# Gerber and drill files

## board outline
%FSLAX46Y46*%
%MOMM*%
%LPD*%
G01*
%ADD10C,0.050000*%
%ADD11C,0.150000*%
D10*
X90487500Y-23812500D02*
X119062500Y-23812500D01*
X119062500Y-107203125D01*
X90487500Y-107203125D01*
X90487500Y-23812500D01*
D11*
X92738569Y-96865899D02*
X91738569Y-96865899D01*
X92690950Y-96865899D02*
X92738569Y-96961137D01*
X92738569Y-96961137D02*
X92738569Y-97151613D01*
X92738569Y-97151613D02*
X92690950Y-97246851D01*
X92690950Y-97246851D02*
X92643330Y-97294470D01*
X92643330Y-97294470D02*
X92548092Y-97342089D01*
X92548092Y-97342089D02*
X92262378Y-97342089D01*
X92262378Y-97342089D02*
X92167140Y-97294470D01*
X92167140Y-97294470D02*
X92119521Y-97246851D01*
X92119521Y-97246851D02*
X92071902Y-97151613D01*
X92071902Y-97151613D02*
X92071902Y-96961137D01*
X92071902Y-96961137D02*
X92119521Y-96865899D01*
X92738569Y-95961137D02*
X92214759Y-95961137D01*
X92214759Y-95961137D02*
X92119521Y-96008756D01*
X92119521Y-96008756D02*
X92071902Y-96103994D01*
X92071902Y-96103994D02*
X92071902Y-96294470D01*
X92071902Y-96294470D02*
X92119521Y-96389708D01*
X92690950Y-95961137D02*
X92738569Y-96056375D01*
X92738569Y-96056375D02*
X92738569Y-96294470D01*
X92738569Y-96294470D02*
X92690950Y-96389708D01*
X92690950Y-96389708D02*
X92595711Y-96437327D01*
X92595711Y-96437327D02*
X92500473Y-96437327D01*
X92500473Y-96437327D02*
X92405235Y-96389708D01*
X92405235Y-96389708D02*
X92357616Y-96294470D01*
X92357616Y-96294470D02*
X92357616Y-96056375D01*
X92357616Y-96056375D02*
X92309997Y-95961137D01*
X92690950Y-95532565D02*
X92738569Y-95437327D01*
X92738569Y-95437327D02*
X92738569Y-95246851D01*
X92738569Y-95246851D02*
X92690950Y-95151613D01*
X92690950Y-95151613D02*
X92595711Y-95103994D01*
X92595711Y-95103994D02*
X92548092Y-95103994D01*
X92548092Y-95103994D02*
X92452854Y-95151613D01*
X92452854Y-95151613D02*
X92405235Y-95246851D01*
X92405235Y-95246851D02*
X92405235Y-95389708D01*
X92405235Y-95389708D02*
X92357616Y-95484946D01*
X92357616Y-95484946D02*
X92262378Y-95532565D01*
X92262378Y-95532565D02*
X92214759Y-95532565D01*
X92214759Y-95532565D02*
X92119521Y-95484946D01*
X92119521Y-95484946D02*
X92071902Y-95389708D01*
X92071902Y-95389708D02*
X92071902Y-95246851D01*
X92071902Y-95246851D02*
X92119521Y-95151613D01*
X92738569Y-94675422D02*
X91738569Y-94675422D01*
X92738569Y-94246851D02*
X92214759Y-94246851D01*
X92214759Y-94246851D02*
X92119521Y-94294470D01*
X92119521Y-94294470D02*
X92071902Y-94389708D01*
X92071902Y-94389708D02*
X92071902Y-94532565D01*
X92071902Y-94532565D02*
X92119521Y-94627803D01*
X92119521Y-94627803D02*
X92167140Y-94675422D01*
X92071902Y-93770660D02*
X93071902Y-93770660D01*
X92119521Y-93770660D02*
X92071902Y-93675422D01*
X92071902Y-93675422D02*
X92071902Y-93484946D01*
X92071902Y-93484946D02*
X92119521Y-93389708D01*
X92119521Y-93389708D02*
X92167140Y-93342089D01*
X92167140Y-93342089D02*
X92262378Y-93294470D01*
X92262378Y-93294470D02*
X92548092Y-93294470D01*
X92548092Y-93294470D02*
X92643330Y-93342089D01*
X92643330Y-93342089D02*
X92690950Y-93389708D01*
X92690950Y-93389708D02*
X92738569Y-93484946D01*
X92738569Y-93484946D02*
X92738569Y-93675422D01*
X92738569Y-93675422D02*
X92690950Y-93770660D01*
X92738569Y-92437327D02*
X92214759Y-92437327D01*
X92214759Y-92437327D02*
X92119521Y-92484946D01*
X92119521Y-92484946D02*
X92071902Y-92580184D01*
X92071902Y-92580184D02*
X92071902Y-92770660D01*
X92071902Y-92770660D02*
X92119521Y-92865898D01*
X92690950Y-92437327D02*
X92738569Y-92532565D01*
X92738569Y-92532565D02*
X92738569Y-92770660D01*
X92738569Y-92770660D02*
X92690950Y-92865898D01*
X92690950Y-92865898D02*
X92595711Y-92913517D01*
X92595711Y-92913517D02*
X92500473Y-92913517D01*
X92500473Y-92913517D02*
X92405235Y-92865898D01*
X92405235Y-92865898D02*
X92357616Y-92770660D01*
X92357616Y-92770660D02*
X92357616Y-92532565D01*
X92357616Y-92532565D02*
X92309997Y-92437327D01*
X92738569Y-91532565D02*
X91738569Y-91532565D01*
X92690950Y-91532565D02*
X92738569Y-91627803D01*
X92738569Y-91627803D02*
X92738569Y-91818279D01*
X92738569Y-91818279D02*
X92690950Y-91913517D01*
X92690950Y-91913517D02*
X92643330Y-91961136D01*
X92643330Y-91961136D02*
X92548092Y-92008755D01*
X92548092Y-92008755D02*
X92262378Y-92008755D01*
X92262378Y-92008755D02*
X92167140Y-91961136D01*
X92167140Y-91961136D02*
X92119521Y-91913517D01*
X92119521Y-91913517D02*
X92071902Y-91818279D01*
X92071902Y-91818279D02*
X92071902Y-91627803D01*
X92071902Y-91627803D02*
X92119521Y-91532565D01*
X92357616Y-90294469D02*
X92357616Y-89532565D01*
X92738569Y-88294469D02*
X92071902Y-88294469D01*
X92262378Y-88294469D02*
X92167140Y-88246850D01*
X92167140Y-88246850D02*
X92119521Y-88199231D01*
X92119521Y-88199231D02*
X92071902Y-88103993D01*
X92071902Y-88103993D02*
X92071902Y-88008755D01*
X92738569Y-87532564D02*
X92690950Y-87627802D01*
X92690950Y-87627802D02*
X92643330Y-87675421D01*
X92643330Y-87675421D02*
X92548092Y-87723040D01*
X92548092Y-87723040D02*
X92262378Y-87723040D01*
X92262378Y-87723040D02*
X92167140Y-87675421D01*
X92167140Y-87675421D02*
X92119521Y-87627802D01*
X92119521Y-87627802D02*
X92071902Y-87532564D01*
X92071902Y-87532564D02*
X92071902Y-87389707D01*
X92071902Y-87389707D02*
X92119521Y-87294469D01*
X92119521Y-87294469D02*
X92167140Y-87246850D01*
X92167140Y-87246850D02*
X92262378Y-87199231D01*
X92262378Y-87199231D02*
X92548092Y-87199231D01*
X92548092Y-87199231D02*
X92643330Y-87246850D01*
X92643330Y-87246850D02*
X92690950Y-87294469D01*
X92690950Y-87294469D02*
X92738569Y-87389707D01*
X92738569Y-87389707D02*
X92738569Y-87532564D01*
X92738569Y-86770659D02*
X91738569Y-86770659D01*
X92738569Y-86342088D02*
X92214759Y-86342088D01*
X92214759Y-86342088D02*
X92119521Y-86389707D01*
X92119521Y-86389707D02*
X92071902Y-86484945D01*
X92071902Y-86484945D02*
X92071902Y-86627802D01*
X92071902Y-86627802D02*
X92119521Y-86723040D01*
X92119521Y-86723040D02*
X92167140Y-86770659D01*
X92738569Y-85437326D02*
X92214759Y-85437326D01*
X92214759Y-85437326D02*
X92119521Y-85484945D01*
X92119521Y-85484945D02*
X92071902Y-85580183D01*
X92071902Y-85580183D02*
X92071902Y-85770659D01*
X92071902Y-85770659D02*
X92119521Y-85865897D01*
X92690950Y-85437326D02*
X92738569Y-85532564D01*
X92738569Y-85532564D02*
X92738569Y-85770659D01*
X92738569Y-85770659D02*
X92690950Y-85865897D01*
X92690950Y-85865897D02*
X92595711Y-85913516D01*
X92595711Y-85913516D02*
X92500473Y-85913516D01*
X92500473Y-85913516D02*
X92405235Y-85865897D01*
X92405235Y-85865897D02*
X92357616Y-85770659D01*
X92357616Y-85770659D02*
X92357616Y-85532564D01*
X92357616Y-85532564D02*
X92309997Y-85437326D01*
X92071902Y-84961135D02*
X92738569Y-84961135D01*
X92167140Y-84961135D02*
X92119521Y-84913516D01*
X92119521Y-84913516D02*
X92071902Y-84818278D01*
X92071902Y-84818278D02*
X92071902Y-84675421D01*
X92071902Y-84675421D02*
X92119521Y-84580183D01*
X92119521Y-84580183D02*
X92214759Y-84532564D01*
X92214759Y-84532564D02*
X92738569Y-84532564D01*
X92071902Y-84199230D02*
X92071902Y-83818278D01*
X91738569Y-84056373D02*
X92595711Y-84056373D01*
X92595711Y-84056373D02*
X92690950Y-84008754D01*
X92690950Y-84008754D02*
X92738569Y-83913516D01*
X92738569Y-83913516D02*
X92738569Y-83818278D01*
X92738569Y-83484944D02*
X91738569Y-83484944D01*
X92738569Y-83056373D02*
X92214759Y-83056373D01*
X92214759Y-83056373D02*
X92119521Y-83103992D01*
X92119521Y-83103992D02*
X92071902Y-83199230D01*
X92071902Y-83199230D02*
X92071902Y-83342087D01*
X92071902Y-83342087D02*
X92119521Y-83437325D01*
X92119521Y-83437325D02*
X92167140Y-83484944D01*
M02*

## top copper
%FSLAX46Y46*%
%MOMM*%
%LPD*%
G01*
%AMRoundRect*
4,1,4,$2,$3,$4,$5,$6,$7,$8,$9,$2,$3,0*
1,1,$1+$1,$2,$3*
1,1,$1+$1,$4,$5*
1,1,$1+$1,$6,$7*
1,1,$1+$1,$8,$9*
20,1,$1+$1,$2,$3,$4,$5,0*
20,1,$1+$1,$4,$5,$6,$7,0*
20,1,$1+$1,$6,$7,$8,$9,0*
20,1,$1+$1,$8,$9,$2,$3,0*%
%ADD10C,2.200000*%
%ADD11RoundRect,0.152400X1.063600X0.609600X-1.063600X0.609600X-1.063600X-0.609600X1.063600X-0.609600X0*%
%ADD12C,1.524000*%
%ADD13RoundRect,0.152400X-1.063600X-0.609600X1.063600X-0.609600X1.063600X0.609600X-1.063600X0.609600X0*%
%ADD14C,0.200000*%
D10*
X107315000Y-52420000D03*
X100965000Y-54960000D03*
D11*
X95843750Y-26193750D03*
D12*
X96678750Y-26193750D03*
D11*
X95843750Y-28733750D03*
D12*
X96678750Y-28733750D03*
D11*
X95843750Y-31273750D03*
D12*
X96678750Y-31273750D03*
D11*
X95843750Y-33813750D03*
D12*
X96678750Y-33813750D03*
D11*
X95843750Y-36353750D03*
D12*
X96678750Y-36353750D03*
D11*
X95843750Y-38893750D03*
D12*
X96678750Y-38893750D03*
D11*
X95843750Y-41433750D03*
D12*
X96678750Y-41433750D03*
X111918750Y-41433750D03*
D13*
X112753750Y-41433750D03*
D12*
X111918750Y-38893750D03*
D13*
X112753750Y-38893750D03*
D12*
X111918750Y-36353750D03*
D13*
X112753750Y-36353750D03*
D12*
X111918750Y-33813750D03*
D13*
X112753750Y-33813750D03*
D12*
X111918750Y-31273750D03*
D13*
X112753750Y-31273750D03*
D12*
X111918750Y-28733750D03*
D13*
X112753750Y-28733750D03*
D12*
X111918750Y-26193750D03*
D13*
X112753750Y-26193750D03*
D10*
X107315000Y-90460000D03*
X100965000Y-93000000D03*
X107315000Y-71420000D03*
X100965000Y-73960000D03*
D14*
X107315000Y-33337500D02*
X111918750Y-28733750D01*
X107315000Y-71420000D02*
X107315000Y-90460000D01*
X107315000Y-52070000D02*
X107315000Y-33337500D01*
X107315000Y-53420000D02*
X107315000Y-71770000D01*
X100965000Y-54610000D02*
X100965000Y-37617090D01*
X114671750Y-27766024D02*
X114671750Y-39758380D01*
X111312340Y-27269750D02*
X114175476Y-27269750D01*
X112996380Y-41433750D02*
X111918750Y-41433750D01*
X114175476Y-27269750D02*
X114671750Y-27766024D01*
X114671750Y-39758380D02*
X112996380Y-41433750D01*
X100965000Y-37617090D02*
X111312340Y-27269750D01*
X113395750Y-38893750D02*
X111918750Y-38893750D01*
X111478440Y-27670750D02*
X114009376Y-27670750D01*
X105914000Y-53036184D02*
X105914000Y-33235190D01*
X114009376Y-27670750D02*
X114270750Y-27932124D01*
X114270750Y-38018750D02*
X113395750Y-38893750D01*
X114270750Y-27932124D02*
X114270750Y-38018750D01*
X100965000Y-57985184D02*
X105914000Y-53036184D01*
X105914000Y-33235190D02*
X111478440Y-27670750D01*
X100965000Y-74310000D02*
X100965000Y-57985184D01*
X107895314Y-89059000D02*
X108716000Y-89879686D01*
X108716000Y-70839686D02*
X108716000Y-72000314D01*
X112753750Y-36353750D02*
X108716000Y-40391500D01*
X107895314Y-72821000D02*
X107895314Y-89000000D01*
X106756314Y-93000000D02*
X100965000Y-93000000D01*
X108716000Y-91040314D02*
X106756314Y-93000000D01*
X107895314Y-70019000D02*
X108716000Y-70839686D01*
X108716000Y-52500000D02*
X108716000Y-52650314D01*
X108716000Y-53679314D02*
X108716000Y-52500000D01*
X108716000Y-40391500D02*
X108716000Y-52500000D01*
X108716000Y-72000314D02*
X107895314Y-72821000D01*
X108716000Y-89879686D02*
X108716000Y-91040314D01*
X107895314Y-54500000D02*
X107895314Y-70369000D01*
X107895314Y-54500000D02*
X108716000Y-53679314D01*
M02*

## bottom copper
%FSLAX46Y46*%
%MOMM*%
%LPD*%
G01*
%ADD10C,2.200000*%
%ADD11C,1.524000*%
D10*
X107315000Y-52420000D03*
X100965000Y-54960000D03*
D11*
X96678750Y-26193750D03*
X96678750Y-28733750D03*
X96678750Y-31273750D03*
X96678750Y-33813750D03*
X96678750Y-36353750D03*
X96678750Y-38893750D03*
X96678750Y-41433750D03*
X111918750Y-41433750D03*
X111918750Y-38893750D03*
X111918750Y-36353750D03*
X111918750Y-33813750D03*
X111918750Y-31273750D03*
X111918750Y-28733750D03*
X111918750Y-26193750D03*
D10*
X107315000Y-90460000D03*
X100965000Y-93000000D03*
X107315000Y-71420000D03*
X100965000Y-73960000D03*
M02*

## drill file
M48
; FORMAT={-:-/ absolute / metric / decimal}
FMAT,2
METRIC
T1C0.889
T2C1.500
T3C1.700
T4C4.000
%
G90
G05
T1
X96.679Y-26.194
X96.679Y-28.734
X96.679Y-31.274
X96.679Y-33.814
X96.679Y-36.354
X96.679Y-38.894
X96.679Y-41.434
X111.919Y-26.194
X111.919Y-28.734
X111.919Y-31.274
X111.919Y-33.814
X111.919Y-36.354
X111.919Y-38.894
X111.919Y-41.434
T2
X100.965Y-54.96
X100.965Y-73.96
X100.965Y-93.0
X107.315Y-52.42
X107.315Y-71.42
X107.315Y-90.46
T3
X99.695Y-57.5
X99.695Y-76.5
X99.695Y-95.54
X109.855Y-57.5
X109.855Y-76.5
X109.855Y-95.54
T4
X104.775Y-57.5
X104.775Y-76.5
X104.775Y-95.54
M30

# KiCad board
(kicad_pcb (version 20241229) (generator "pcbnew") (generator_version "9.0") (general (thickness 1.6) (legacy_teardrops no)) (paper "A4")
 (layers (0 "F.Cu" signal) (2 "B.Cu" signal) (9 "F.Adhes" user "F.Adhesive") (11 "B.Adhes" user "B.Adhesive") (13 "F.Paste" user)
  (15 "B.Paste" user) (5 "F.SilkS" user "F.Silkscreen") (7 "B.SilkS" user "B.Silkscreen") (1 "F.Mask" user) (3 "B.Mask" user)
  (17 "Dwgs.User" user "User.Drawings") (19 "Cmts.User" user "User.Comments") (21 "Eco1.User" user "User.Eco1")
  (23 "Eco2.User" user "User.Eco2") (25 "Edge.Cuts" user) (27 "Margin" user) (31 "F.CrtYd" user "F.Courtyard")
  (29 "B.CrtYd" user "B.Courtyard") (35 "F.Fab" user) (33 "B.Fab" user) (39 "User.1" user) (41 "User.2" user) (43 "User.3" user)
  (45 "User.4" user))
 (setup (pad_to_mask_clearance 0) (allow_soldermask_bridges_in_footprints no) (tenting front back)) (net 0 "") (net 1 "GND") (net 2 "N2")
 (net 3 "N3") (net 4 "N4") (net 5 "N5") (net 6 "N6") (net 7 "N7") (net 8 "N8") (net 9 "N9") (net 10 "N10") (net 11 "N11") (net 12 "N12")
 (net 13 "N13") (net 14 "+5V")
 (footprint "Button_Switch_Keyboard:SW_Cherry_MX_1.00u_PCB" (layer "F.Cu") (at 107.315 52.42)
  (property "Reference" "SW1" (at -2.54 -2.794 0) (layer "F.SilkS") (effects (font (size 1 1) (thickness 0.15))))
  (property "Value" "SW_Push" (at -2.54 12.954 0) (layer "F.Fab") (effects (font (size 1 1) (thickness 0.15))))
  (pad "" np_thru_hole circle (at -7.62 5.08) (size 1.7 1.7) (drill 1.7) (layers "*.Cu" "*.Mask"))
  (pad "" np_thru_hole circle (at -2.54 5.08) (size 4 4) (drill 4) (layers "*.Cu" "*.Mask"))
  (pad "" np_thru_hole circle (at 2.54 5.08) (size 1.7 1.7) (drill 1.7) (layers "*.Cu" "*.Mask"))
  (pad "1" thru_hole circle (at 0 0) (size 2.2 2.2) (drill 1.5) (layers "*.Cu" "*.Mask") (remove_unused_layers no) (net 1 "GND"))
  (pad "2" thru_hole circle (at -6.35 2.54) (size 2.2 2.2) (drill 1.5) (layers "*.Cu" "*.Mask") (remove_unused_layers no) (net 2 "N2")))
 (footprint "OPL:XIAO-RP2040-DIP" (layer "F.Cu") (at 104.29875 33.81375)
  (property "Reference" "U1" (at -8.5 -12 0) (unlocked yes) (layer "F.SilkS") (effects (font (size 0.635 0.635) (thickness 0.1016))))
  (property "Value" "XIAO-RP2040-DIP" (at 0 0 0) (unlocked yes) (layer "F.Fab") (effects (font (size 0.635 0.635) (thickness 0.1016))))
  (pad "1" smd roundrect (at -8.455 -7.62 180) (size 2.432 1.524) (layers "F.Cu" "F.Mask") (roundrect_rratio 0.1) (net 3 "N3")
   (thermal_bridge_angle 45))
  (pad "1" thru_hole circle (at -7.62 -7.62 180) (size 1.524 1.524) (drill 0.889) (layers "*.Cu" "*.Mask") (remove_unused_layers no)
   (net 3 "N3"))
  (pad "2" smd roundrect (at -8.455 -5.08 180) (size 2.432 1.524) (layers "F.Cu" "F.Mask") (roundrect_rratio 0.1) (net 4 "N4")
   (thermal_bridge_angle 45))
  (pad "2" thru_hole circle (at -7.62 -5.08 180) (size 1.524 1.524) (drill 0.889) (layers "*.Cu" "*.Mask") (remove_unused_layers no)
   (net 4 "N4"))
  (pad "3" smd roundrect (at -8.455 -2.54 180) (size 2.432 1.524) (layers "F.Cu" "F.Mask") (roundrect_rratio 0.1) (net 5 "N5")
   (thermal_bridge_angle 45))
  (pad "3" thru_hole circle (at -7.62 -2.54 180) (size 1.524 1.524) (drill 0.889) (layers "*.Cu" "*.Mask") (remove_unused_layers no)
   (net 5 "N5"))
  (pad "4" smd roundrect (at -8.455 0 180) (size 2.432 1.524) (layers "F.Cu" "F.Mask") (roundrect_rratio 0.1) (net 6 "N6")
   (thermal_bridge_angle 45))
  (pad "4" thru_hole circle (at -7.62 0 180) (size 1.524 1.524) (drill 0.889) (layers "*.Cu" "*.Mask") (remove_unused_layers no)
   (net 6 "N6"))
  (pad "5" smd roundrect (at -8.455 2.54 180) (size 2.432 1.524) (layers "F.Cu" "F.Mask") (roundrect_rratio 0.1) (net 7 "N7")
   (thermal_bridge_angle 45))
  (pad "5" thru_hole circle (at -7.62 2.54 180) (size 1.524 1.524) (drill 0.889) (layers "*.Cu" "*.Mask") (remove_unused_layers no)
   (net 7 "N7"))
  (pad "6" smd roundrect (at -8.455 5.08 180) (size 2.432 1.524) (layers "F.Cu" "F.Mask") (roundrect_rratio 0.1) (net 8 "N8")
   (thermal_bridge_angle 45))
  (pad "6" thru_hole circle (at -7.62 5.08 180) (size 1.524 1.524) (drill 0.889) (layers "*.Cu" "*.Mask") (remove_unused_layers no)
   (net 8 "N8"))
  (pad "7" smd roundrect (at -8.455 7.62 180) (size 2.432 1.524) (layers "F.Cu" "F.Mask") (roundrect_rratio 0.1) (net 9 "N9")
   (thermal_bridge_angle 45))
  (pad "7" thru_hole circle (at -7.62 7.62 180) (size 1.524 1.524) (drill 0.889) (layers "*.Cu" "*.Mask") (remove_unused_layers no)
   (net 9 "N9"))
  (pad "8" thru_hole circle (at 7.62 7.62) (size 1.524 1.524) (drill 0.889) (layers "*.Cu" "*.Mask") (remove_unused_layers no) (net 2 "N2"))
  (pad "8" smd roundrect (at 8.455 7.62) (size 2.432 1.524) (layers "F.Cu" "F.Mask") (roundrect_rratio 0.1) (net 2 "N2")
   (thermal_bridge_angle 45))
  (pad "9" thru_hole circle (at 7.62 5.08) (size 1.524 1.524) (drill 0.889) (layers "*.Cu" "*.Mask") (remove_unused_layers no)
   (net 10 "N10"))
  (pad "9" smd roundrect (at 8.455 5.08) (size 2.432 1.524) (layers "F.Cu" "F.Mask") (roundrect_rratio 0.1) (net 10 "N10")
   (thermal_bridge_angle 45))
  (pad "10" thru_hole circle (at 7.62 2.54) (size 1.524 1.524) (drill 0.889) (layers "*.Cu" "*.Mask") (remove_unused_layers no)
   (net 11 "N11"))
  (pad "10" smd roundrect (at 8.455 2.54) (size 2.432 1.524) (layers "F.Cu" "F.Mask") (roundrect_rratio 0.1) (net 11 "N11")
   (thermal_bridge_angle 45))
  (pad "11" thru_hole circle (at 7.62 0) (size 1.524 1.524) (drill 0.889) (layers "*.Cu" "*.Mask") (remove_unused_layers no) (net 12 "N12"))
  (pad "11" smd roundrect (at 8.455 0) (size 2.432 1.524) (layers "F.Cu" "F.Mask") (roundrect_rratio 0.1) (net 12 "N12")
   (thermal_bridge_angle 45))
  (pad "12" thru_hole circle (at 7.62 -2.54) (size 1.524 1.524) (drill 0.889) (layers "*.Cu" "*.Mask") (remove_unused_layers no)
   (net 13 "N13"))
  (pad "12" smd roundrect (at 8.455 -2.54) (size 2.432 1.524) (layers "F.Cu" "F.Mask") (roundrect_rratio 0.1) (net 13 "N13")
   (thermal_bridge_angle 45))
  (pad "13" thru_hole circle (at 7.62 -5.08) (size 1.524 1.524) (drill 0.889) (layers "*.Cu" "*.Mask") (remove_unused_layers no)
   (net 1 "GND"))
  (pad "13" smd roundrect (at 8.455 -5.08) (size 2.432 1.524) (layers "F.Cu" "F.Mask") (roundrect_rratio 0.1) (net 1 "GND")
   (thermal_bridge_angle 45))
  (pad "14" thru_hole circle (at 7.62 -7.62) (size 1.524 1.524) (drill 0.889) (layers "*.Cu" "*.Mask") (remove_unused_layers no)
   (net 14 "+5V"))
  (pad "14" smd roundrect (at 8.455 -7.62) (size 2.432 1.524) (layers "F.Cu" "F.Mask") (roundrect_rratio 0.1) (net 14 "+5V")
   (thermal_bridge_angle 45)))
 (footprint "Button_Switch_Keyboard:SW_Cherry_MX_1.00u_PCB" (layer "F.Cu") (at 107.315 90.46)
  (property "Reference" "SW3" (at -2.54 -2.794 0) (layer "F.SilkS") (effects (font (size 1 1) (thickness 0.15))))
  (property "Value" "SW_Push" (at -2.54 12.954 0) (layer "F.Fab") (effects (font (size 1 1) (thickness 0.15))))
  (pad "" np_thru_hole circle (at -7.62 5.08) (size 1.7 1.7) (drill 1.7) (layers "*.Cu" "*.Mask"))
  (pad "" np_thru_hole circle (at -2.54 5.08) (size 4 4) (drill 4) (layers "*.Cu" "*.Mask"))
  (pad "" np_thru_hole circle (at 2.54 5.08) (size 1.7 1.7) (drill 1.7) (layers "*.Cu" "*.Mask"))
  (pad "1" thru_hole circle (at 0 0) (size 2.2 2.2) (drill 1.5) (layers "*.Cu" "*.Mask") (remove_unused_layers no) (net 1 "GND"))
  (pad "2" thru_hole circle (at -6.35 2.54) (size 2.2 2.2) (drill 1.5) (layers "*.Cu" "*.Mask") (remove_unused_layers no) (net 11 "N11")))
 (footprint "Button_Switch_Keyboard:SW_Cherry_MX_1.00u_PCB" (layer "F.Cu") (at 107.315 71.42)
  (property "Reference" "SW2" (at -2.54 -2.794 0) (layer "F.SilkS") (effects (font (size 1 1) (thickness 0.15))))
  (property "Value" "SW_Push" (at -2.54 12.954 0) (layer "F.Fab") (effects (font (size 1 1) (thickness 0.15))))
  (pad "" np_thru_hole circle (at -7.62 5.08) (size 1.7 1.7) (drill 1.7) (layers "*.Cu" "*.Mask"))
  (pad "" np_thru_hole circle (at -2.54 5.08) (size 4 4) (drill 4) (layers "*.Cu" "*.Mask"))
  (pad "" np_thru_hole circle (at 2.54 5.08) (size 1.7 1.7) (drill 1.7) (layers "*.Cu" "*.Mask"))
  (pad "1" thru_hole circle (at 0 0) (size 2.2 2.2) (drill 1.5) (layers "*.Cu" "*.Mask") (remove_unused_layers no) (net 1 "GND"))
  (pad "2" thru_hole circle (at -6.35 2.54) (size 2.2 2.2) (drill 1.5) (layers "*.Cu" "*.Mask") (remove_unused_layers no) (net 10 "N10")))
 (gr_rect (start 90.4875 23.8125) (end 119.0625 107.203125) (stroke (width 0.05) (type default)) (fill no) (layer "Edge.Cuts"))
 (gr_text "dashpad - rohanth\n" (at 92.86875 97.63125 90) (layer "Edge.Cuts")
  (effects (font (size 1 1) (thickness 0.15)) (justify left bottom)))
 (segment (start 107.315 33.3375) (end 111.91875 28.73375) (width 0.2) (layer "F.Cu") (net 1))
 (segment (start 107.315 71.42) (end 107.315 90.46) (width 0.2) (layer "F.Cu") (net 1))
 (segment (start 107.315 52.07) (end 107.315 33.3375) (width 0.2) (layer "F.Cu") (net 1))
 (segment (start 107.315 53.42) (end 107.315 71.77) (width 0.2) (layer "F.Cu") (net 1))
 (segment (start 100.965 54.61) (end 100.965 37.61709) (width 0.2) (layer "F.Cu") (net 2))
 (segment (start 114.67175 27.766024) (end 114.67175 39.75838) (width 0.2) (layer "F.Cu") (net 2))
 (segment (start 111.31234 27.26975) (end 114.175476 27.26975) (width 0.2) (layer "F.Cu") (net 2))
 (segment (start 112.99638 41.43375) (end 111.91875 41.43375) (width 0.2) (layer "F.Cu") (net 2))
 (segment (start 114.175476 27.26975) (end 114.67175 27.766024) (width 0.2) (layer "F.Cu") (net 2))
 (segment (start 114.67175 39.75838) (end 112.99638 41.43375) (width 0.2) (layer "F.Cu") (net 2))
 (segment (start 100.965 37.61709) (end 111.31234 27.26975) (width 0.2) (layer "F.Cu") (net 2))
 (segment (start 113.39575 38.89375) (end 111.91875 38.89375) (width 0.2) (layer "F.Cu") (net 10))
 (segment (start 111.47844 27.67075) (end 114.009376 27.67075) (width 0.2) (layer "F.Cu") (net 10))
 (segment (start 105.914 53.036184) (end 105.914 33.23519) (width 0.2) (layer "F.Cu") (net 10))
 (segment (start 114.009376 27.67075) (end 114.27075 27.932124) (width 0.2) (layer "F.Cu") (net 10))
 (segment (start 114.27075 38.01875) (end 113.39575 38.89375) (width 0.2) (layer "F.Cu") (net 10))
 (segment (start 114.27075 27.932124) (end 114.27075 38.01875) (width 0.2) (layer "F.Cu") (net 10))
 (segment (start 100.965 57.985184) (end 105.914 53.036184) (width 0.2) (layer "F.Cu") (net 10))
 (segment (start 105.914 33.23519) (end 111.47844 27.67075) (width 0.2) (layer "F.Cu") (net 10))
 (segment (start 100.965 74.31) (end 100.965 57.985184) (width 0.2) (layer "F.Cu") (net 10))
 (segment (start 107.895314 89.059) (end 108.716 89.879686) (width 0.2) (layer "F.Cu") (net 11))
 (segment (start 108.716 70.839686) (end 108.716 72.000314) (width 0.2) (layer "F.Cu") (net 11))
 (segment (start 112.75375 36.35375) (end 108.716 40.3915) (width 0.2) (layer "F.Cu") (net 11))
 (segment (start 107.895314 72.821) (end 107.895314 89) (width 0.2) (layer "F.Cu") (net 11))
 (segment (start 106.756314 93) (end 100.965 93) (width 0.2) (layer "F.Cu") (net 11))
 (segment (start 108.716 91.040314) (end 106.756314 93) (width 0.2) (layer "F.Cu") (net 11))
 (segment (start 107.895314 70.019) (end 108.716 70.839686) (width 0.2) (layer "F.Cu") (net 11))
 (segment (start 108.716 52.5) (end 108.716 52.650314) (width 0.2) (layer "F.Cu") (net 11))
 (segment (start 108.716 53.679314) (end 108.716 52.5) (width 0.2) (layer "F.Cu") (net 11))
 (segment (start 108.716 40.3915) (end 108.716 52.5) (width 0.2) (layer "F.Cu") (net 11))
 (segment (start 108.716 72.000314) (end 107.895314 72.821) (width 0.2) (layer "F.Cu") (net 11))
 (segment (start 108.716 89.879686) (end 108.716 91.040314) (width 0.2) (layer "F.Cu") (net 11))
 (segment (start 107.895314 54.5) (end 107.895314 70.369) (width 0.2) (layer "F.Cu") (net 11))
 (segment (start 107.895314 54.5) (end 108.716 53.679314) (width 0.2) (layer "F.Cu") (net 11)))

